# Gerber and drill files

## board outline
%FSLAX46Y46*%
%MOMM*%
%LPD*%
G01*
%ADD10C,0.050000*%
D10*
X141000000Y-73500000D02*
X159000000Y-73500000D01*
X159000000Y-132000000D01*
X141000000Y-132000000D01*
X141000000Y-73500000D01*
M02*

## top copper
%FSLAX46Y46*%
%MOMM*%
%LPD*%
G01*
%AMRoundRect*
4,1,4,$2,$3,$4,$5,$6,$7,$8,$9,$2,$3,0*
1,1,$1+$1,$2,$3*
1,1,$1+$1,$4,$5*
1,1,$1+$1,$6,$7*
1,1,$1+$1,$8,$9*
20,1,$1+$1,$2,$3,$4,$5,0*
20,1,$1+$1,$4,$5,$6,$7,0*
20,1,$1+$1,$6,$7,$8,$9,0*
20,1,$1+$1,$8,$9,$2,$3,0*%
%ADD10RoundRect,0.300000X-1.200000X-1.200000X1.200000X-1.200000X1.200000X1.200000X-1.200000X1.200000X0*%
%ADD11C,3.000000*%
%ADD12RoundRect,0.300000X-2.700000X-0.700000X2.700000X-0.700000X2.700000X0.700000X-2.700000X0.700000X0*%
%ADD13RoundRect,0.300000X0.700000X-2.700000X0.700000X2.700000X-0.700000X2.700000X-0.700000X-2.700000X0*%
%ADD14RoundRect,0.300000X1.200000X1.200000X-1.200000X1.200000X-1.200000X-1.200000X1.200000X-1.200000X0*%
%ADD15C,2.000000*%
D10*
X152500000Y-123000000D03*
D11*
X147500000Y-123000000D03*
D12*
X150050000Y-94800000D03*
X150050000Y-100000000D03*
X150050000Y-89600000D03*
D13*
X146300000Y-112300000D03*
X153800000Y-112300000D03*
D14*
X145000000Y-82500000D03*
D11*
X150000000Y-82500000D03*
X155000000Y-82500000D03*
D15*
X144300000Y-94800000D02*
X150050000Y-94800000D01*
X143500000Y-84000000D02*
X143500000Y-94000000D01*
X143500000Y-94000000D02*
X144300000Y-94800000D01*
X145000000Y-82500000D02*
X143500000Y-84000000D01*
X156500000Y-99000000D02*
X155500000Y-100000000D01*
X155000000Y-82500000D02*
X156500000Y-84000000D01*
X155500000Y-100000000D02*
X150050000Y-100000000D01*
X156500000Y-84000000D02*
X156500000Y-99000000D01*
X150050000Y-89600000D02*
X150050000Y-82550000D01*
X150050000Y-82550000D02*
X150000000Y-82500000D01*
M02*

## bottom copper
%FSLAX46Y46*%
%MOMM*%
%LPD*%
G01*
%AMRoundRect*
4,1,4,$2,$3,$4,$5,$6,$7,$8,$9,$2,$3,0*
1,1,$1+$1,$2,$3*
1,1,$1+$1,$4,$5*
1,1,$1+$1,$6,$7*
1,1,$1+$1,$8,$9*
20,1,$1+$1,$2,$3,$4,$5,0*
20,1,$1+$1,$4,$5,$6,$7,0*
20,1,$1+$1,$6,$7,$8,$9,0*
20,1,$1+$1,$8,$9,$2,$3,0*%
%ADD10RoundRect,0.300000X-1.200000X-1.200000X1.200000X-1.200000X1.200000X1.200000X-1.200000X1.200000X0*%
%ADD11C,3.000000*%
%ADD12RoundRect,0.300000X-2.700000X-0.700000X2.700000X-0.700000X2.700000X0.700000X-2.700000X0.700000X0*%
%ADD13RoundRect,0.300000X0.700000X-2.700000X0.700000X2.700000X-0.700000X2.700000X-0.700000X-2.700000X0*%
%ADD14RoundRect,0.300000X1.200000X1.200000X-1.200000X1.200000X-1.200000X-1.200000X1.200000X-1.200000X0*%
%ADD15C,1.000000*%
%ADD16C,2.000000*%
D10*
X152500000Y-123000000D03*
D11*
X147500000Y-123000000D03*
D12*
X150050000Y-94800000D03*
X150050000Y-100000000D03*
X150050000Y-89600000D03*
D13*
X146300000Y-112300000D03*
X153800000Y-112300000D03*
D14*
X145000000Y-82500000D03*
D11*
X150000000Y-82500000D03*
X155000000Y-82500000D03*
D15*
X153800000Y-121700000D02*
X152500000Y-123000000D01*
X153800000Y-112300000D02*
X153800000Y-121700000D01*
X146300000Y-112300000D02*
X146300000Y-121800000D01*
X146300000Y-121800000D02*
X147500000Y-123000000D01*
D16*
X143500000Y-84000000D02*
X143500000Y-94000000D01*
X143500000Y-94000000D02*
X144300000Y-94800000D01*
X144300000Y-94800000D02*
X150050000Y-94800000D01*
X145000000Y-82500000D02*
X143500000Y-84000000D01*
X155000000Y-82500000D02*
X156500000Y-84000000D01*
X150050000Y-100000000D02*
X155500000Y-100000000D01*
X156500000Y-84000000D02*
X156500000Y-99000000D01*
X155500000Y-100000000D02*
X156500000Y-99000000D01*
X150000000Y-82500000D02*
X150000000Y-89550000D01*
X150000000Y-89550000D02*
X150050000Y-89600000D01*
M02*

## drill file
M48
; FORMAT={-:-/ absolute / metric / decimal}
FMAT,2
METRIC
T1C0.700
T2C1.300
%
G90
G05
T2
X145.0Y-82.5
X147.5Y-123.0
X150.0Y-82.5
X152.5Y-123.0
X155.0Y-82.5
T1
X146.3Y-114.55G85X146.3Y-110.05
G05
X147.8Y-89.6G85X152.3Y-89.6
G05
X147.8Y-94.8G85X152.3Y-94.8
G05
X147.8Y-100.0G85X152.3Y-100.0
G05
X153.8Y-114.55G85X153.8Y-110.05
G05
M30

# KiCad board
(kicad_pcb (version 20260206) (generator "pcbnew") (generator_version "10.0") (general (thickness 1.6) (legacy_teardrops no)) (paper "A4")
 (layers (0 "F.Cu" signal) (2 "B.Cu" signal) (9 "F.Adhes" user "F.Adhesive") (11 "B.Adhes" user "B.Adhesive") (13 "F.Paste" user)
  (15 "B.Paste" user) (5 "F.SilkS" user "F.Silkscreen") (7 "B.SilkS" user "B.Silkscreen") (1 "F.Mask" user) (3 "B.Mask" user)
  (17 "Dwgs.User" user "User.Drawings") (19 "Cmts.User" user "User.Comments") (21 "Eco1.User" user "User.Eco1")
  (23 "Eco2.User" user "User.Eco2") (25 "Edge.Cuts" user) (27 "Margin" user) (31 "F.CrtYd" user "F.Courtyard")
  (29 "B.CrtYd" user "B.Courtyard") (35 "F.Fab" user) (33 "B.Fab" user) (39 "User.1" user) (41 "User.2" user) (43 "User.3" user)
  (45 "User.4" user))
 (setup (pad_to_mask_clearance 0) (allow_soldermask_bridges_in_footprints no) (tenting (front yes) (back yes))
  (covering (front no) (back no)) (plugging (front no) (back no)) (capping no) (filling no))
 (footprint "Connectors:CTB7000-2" (layer "F.Cu") (at 150 123)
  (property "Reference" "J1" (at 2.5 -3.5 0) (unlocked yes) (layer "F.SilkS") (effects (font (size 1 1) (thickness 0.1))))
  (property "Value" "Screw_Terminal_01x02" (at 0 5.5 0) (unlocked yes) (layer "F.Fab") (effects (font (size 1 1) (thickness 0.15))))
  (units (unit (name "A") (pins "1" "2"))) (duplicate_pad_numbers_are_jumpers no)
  (pad "1" thru_hole roundrect (at 2.5 0) (size 3 3) (drill 1.3) (layers "*.Cu" "*.Mask") (remove_unused_layers no) (roundrect_rratio 0.1)
   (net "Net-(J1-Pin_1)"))
  (pad "2" thru_hole circle (at -2.5 0) (size 3 3) (drill 1.3) (layers "*.Cu" "*.Mask") (remove_unused_layers no) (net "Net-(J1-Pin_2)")))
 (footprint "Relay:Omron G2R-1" (layer "F.Cu") (at 150.05 94.8)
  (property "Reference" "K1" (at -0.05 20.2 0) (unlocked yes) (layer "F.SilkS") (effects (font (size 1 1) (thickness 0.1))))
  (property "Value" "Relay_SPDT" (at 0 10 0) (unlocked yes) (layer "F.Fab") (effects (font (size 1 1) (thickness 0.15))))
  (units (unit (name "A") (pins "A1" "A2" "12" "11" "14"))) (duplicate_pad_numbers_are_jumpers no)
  (pad "11" thru_hole roundrect (at 0 0) (size 6 2) (drill oval 5.2 0.7) (layers "*.Cu" "*.Mask") (remove_unused_layers no)
   (roundrect_rratio 0.15) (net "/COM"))
  (pad "12" thru_hole roundrect (at 0 5.2) (size 6 2) (drill oval 5.2 0.7) (layers "*.Cu" "*.Mask") (remove_unused_layers no)
   (roundrect_rratio 0.15) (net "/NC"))
  (pad "14" thru_hole roundrect (at 0 -5.2) (size 6 2) (drill oval 5.2 0.7) (layers "*.Cu" "*.Mask") (remove_unused_layers no)
   (roundrect_rratio 0.15) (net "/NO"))
  (pad "A1" thru_hole roundrect (at -3.75 17.5 90) (size 6 2) (drill oval 5.2 0.7) (layers "*.Cu" "*.Mask") (remove_unused_layers no)
   (roundrect_rratio 0.15) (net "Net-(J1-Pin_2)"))
  (pad "A2" thru_hole roundrect (at 3.75 17.5 90) (size 6 2) (drill oval 5.2 0.7) (layers "*.Cu" "*.Mask") (remove_unused_layers no)
   (roundrect_rratio 0.15) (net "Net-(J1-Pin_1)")))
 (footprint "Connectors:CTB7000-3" (layer "F.Cu") (at 150 82.5 180)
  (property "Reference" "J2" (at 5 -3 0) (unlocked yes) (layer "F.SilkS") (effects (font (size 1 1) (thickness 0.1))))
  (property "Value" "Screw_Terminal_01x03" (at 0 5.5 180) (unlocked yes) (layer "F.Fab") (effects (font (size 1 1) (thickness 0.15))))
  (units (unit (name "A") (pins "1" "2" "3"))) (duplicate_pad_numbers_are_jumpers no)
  (pad "1" thru_hole roundrect (at 5 0 180) (size 3 3) (drill 1.3) (layers "*.Cu" "*.Mask") (remove_unused_layers no) (roundrect_rratio 0.1)
   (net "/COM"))
  (pad "2" thru_hole circle (at 0 0 180) (size 3 3) (drill 1.3) (layers "*.Cu" "*.Mask") (remove_unused_layers no) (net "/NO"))
  (pad "3" thru_hole circle (at -5 0 180) (size 3 3) (drill 1.3) (layers "*.Cu" "*.Mask") (remove_unused_layers no) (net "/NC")))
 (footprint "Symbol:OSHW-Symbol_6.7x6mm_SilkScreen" (layer "B.Cu") (at 145 128.5 180)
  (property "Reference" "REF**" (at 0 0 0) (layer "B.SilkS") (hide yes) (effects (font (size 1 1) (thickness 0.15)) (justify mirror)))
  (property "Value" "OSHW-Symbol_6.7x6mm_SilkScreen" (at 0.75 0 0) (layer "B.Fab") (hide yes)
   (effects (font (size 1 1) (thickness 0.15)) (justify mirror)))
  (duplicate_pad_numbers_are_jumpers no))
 (gr_rect (start 141 73.5) (end 159 132) (stroke (width 0.05) (type default)) (fill no) (layer "Edge.Cuts"))
 (segment (start 153.8 121.7) (end 152.5 123) (width 1) (layer "B.Cu") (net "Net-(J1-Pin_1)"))
 (segment (start 153.8 112.3) (end 153.8 121.7) (width 1) (layer "B.Cu") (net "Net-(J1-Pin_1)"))
 (segment (start 146.3 112.3) (end 146.3 121.8) (width 1) (layer "B.Cu") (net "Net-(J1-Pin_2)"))
 (segment (start 146.3 121.8) (end 147.5 123) (width 1) (layer "B.Cu") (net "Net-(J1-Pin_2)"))
 (segment (start 144.3 94.8) (end 150.05 94.8) (width 2) (layer "F.Cu") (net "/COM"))
 (segment (start 143.5 84) (end 143.5 94) (width 2) (layer "F.Cu") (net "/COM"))
 (segment (start 143.5 94) (end 144.3 94.8) (width 2) (layer "F.Cu") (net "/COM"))
 (segment (start 145 82.5) (end 143.5 84) (width 2) (layer "F.Cu") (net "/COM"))
 (segment (start 143.5 84) (end 143.5 94) (width 2) (locked yes) (layer "B.Cu") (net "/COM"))
 (segment (start 143.5 94) (end 144.3 94.8) (width 2) (locked yes) (layer "B.Cu") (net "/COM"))
 (segment (start 144.3 94.8) (end 150.05 94.8) (width 2) (locked yes) (layer "B.Cu") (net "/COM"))
 (segment (start 145 82.5) (end 143.5 84) (width 2) (locked yes) (layer "B.Cu") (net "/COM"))
 (segment (start 156.5 99) (end 155.5 100) (width 2) (layer "F.Cu") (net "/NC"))
 (segment (start 155 82.5) (end 156.5 84) (width 2) (layer "F.Cu") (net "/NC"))
 (segment (start 155.5 100) (end 150.05 100) (width 2) (layer "F.Cu") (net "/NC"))
 (segment (start 156.5 84) (end 156.5 99) (width 2) (layer "F.Cu") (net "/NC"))
 (segment (start 155 82.5) (end 156.5 84) (width 2) (locked yes) (layer "B.Cu") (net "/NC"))
 (segment (start 150.05 100) (end 155.5 100) (width 2) (locked yes) (layer "B.Cu") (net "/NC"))
 (segment (start 156.5 84) (end 156.5 99) (width 2) (locked yes) (layer "B.Cu") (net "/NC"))
 (segment (start 155.5 100) (end 156.5 99) (width 2) (locked yes) (layer "B.Cu") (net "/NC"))
 (segment (start 150.05 89.6) (end 150.05 82.55) (width 2) (layer "F.Cu") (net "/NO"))
 (segment (start 150.05 82.55) (end 150 82.5) (width 2) (layer "F.Cu") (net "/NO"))
 (segment (start 150 82.5) (end 150 89.55) (width 2) (locked yes) (layer "B.Cu") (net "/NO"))
 (segment (start 150 89.55) (end 150.05 89.6) (width 2) (layer "B.Cu") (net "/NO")))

